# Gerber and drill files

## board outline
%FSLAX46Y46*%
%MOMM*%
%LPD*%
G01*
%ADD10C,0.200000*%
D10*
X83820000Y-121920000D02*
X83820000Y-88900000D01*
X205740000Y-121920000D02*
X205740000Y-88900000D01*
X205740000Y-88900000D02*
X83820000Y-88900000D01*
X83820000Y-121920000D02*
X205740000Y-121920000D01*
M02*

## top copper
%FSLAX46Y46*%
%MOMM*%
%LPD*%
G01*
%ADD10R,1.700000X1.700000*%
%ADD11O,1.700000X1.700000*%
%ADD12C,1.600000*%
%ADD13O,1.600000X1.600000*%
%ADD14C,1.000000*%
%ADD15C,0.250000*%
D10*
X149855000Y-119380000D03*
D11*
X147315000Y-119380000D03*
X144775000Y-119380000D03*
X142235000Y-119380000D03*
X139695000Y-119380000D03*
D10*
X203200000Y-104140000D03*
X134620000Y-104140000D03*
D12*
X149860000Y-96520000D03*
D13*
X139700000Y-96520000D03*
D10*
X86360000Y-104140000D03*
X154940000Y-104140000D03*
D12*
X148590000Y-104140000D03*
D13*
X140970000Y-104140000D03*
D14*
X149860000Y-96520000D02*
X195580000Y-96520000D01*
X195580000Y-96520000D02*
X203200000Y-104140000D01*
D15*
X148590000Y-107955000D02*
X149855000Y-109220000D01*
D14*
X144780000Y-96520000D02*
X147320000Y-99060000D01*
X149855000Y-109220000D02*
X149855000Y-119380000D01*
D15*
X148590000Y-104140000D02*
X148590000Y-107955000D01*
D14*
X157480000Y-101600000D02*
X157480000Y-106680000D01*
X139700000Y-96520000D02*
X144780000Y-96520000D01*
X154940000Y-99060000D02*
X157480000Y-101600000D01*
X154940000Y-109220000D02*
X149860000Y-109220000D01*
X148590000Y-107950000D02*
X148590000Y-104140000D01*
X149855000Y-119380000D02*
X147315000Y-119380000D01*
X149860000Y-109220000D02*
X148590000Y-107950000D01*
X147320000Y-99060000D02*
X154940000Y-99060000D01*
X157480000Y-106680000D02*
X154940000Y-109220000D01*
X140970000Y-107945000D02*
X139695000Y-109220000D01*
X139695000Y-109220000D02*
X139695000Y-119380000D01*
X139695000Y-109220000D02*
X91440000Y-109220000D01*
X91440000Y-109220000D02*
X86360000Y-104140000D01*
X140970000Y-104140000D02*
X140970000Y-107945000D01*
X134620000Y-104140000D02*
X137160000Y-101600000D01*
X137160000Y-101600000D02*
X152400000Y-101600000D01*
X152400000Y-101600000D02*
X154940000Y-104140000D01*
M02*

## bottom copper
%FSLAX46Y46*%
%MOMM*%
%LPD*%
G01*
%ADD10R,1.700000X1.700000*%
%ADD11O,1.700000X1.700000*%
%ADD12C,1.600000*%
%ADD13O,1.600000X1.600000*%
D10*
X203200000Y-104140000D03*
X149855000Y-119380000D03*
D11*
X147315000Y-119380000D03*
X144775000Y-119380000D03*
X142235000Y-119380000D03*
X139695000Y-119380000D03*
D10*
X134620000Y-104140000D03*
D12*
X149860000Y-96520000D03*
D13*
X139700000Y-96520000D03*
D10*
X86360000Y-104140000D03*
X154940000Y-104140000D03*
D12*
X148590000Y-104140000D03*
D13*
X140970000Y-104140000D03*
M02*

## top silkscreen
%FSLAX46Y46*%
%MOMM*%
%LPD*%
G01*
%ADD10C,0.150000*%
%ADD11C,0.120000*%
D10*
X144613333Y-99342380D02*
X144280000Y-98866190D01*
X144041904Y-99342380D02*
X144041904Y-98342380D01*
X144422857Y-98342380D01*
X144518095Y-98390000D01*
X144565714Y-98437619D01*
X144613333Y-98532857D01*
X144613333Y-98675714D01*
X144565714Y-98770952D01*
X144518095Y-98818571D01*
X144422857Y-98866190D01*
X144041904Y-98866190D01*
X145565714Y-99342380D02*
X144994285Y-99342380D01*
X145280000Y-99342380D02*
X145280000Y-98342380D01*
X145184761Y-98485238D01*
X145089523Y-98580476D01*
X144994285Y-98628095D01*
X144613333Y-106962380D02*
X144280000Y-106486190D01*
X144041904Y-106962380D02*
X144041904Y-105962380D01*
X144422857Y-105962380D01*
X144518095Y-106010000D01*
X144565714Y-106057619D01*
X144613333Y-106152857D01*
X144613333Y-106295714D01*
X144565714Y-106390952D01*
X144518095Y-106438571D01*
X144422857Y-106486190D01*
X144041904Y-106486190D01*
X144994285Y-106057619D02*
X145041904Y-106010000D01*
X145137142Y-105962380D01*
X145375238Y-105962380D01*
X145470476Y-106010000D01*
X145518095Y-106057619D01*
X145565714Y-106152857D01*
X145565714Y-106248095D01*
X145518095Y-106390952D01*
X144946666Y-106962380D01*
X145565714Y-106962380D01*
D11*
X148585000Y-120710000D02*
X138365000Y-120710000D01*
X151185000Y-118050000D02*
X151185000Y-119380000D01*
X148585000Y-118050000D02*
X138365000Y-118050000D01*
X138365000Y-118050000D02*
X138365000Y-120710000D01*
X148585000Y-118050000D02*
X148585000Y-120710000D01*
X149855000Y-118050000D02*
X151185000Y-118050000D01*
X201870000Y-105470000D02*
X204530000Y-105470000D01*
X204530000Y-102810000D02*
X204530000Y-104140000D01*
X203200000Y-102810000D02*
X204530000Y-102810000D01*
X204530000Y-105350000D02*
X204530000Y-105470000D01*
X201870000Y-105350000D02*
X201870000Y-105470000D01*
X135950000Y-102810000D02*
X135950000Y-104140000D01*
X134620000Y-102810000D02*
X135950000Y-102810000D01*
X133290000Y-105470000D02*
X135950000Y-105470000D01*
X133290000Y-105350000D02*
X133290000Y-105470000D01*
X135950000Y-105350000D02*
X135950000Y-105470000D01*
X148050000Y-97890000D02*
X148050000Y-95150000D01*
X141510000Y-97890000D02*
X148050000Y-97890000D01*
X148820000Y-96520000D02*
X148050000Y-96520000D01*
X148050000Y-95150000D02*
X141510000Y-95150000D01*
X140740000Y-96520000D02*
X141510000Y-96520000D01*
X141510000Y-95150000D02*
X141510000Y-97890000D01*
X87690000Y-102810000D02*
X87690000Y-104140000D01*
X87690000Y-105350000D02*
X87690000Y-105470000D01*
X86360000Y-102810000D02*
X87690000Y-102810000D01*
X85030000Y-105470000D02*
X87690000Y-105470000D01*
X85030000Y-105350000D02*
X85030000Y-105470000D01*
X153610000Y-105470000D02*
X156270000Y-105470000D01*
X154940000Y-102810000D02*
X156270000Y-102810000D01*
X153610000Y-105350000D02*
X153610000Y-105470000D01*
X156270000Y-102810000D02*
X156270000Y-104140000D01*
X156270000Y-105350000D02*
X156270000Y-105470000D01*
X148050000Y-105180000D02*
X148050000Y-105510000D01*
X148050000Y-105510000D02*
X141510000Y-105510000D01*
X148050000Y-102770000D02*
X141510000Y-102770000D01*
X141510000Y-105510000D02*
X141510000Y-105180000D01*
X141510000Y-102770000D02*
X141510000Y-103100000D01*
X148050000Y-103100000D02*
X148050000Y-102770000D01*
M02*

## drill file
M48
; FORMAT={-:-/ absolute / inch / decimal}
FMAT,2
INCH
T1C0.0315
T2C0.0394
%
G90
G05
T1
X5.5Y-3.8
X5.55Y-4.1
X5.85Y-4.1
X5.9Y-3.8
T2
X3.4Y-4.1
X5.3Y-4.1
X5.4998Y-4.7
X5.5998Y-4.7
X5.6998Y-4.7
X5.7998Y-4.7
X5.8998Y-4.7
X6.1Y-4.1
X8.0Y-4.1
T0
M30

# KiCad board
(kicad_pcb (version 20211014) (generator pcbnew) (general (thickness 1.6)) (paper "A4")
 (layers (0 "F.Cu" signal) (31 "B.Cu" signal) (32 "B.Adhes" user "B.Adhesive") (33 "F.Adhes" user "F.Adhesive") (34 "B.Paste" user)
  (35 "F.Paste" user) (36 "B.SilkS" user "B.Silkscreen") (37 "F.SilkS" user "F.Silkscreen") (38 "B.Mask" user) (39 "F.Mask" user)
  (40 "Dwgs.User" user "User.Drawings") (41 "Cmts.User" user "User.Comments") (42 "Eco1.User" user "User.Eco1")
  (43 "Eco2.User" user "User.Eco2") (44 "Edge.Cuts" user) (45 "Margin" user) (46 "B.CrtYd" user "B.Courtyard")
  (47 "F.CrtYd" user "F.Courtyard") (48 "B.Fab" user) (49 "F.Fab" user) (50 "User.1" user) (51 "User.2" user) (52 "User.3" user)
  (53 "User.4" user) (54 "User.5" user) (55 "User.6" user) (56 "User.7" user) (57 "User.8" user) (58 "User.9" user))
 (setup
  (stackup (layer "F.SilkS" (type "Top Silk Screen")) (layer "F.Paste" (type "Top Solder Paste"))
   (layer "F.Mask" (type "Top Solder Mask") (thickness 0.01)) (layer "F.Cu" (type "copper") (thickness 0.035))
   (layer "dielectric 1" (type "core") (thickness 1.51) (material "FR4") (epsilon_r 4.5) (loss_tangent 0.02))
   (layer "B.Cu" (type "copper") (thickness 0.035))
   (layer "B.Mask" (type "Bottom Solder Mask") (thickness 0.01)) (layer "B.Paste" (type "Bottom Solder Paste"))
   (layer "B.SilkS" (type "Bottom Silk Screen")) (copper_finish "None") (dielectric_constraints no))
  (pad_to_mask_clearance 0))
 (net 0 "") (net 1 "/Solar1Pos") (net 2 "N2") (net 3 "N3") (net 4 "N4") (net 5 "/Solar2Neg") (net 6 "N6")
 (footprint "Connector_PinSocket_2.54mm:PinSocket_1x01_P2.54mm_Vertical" (layer "F.Cu") (at 203.2 104.14)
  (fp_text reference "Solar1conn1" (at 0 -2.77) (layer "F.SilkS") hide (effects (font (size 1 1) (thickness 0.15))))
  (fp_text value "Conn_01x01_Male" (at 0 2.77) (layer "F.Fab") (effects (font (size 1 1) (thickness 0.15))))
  (fp_line (start -1.33 1.33) (end 1.33 1.33) (layer "F.SilkS") (width 0.12))
  (fp_line (start 1.33 -1.33) (end 1.33 0) (layer "F.SilkS") (width 0.12))
  (fp_line (start 0 -1.33) (end 1.33 -1.33) (layer "F.SilkS") (width 0.12))
  (fp_line (start 1.33 1.21) (end 1.33 1.33) (layer "F.SilkS") (width 0.12))
  (fp_line (start -1.33 1.21) (end -1.33 1.33) (layer "F.SilkS") (width 0.12))
  (pad "1" thru_hole rect (at 0 0) (size 1.7 1.7) (drill 1) (layers *.Cu *.Mask) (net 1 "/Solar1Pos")))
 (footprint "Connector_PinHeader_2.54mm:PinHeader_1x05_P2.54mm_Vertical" (layer "F.Cu") (at 149.855 119.38 -90)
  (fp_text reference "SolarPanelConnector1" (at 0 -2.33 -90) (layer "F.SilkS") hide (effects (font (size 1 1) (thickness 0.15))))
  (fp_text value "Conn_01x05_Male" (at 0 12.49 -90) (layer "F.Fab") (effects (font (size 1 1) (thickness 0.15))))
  (fp_line (start -1.33 0) (end -1.33 -1.33) (layer "F.SilkS") (width 0.12))
  (fp_line (start 1.33 1.27) (end 1.33 11.49) (layer "F.SilkS") (width 0.12))
  (fp_line (start -1.33 11.49) (end 1.33 11.49) (layer "F.SilkS") (width 0.12))
  (fp_line (start -1.33 1.27) (end -1.33 11.49) (layer "F.SilkS") (width 0.12))
  (fp_line (start -1.33 1.27) (end 1.33 1.27) (layer "F.SilkS") (width 0.12))
  (fp_line (start -1.33 -1.33) (end 0 -1.33) (layer "F.SilkS") (width 0.12))
  (pad "1" thru_hole rect (at 0 0 270) (size 1.7 1.7) (drill 1) (layers *.Cu *.Mask) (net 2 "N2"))
  (pad "2" thru_hole oval (at 0 2.54 270) (size 1.7 1.7) (drill 1) (layers *.Cu *.Mask) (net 2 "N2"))
  (pad "3" thru_hole oval (at 0 5.08 270) (size 1.7 1.7) (drill 1) (layers *.Cu *.Mask) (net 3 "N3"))
  (pad "4" thru_hole oval (at 0 7.62 270) (size 1.7 1.7) (drill 1) (layers *.Cu *.Mask) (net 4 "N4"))
  (pad "5" thru_hole oval (at 0 10.16 270) (size 1.7 1.7) (drill 1) (layers *.Cu *.Mask) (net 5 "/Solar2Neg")))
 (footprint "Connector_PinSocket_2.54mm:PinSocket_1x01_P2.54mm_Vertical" (layer "F.Cu") (at 134.62 104.14)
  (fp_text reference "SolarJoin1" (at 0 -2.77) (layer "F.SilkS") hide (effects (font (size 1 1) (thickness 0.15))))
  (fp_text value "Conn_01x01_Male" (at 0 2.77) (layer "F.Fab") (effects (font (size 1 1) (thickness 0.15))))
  (fp_line (start 1.33 -1.33) (end 1.33 0) (layer "F.SilkS") (width 0.12))
  (fp_line (start 0 -1.33) (end 1.33 -1.33) (layer "F.SilkS") (width 0.12))
  (fp_line (start -1.33 1.33) (end 1.33 1.33) (layer "F.SilkS") (width 0.12))
  (fp_line (start -1.33 1.21) (end -1.33 1.33) (layer "F.SilkS") (width 0.12))
  (fp_line (start 1.33 1.21) (end 1.33 1.33) (layer "F.SilkS") (width 0.12))
  (pad "1" thru_hole rect (at 0 0) (size 1.7 1.7) (drill 1) (layers *.Cu *.Mask) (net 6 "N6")))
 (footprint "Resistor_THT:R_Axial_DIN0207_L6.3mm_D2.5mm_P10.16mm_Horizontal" (layer "F.Cu") (at 149.86 96.52 180)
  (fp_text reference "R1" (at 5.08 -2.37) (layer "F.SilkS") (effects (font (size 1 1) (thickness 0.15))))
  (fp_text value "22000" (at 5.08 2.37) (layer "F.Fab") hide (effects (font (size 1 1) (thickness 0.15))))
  (fp_line (start 1.81 -1.37) (end 1.81 1.37) (layer "F.SilkS") (width 0.12))
  (fp_line (start 8.35 -1.37) (end 1.81 -1.37) (layer "F.SilkS") (width 0.12))
  (fp_line (start 1.04 0) (end 1.81 0) (layer "F.SilkS") (width 0.12))
  (fp_line (start 1.81 1.37) (end 8.35 1.37) (layer "F.SilkS") (width 0.12))
  (fp_line (start 9.12 0) (end 8.35 0) (layer "F.SilkS") (width 0.12))
  (fp_line (start 8.35 1.37) (end 8.35 -1.37) (layer "F.SilkS") (width 0.12))
  (pad "1" thru_hole circle (at 0 0 180) (size 1.6 1.6) (drill 0.8) (layers *.Cu *.Mask) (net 1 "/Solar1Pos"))
  (pad "2" thru_hole oval (at 10.16 0 180) (size 1.6 1.6) (drill 0.8) (layers *.Cu *.Mask) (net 2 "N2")))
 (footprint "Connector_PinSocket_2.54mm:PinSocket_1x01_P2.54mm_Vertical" (layer "F.Cu") (at 86.36 104.14)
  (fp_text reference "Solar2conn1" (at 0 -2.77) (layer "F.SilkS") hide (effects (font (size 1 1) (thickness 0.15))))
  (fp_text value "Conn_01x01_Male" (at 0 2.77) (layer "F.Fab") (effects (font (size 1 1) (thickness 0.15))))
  (fp_line (start 1.33 -1.33) (end 1.33 0) (layer "F.SilkS") (width 0.12))
  (fp_line (start 1.33 1.21) (end 1.33 1.33) (layer "F.SilkS") (width 0.12))
  (fp_line (start 0 -1.33) (end 1.33 -1.33) (layer "F.SilkS") (width 0.12))
  (fp_line (start -1.33 1.33) (end 1.33 1.33) (layer "F.SilkS") (width 0.12))
  (fp_line (start -1.33 1.21) (end -1.33 1.33) (layer "F.SilkS") (width 0.12))
  (pad "1" thru_hole rect (at 0 0) (size 1.7 1.7) (drill 1) (layers *.Cu *.Mask) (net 5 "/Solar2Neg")))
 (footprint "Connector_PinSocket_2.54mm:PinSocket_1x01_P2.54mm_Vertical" (layer "F.Cu") (at 154.94 104.14)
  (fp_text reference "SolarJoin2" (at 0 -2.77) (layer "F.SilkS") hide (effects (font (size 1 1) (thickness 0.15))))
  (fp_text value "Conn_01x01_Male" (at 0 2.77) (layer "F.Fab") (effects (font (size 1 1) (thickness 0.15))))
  (fp_line (start -1.33 1.33) (end 1.33 1.33) (layer "F.SilkS") (width 0.12))
  (fp_line (start 0 -1.33) (end 1.33 -1.33) (layer "F.SilkS") (width 0.12))
  (fp_line (start -1.33 1.21) (end -1.33 1.33) (layer "F.SilkS") (width 0.12))
  (fp_line (start 1.33 -1.33) (end 1.33 0) (layer "F.SilkS") (width 0.12))
  (fp_line (start 1.33 1.21) (end 1.33 1.33) (layer "F.SilkS") (width 0.12))
  (pad "1" thru_hole rect (at 0 0) (size 1.7 1.7) (drill 1) (layers *.Cu *.Mask) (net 6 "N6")))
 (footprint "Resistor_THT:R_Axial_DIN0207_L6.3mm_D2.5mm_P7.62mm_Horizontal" (layer "F.Cu") (at 148.59 104.14 180)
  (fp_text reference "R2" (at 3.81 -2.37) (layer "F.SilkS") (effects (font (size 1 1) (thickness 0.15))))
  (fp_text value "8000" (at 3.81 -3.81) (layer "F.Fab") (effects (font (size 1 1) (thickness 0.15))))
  (fp_line (start 0.54 -1.04) (end 0.54 -1.37) (layer "F.SilkS") (width 0.12))
  (fp_line (start 0.54 -1.37) (end 7.08 -1.37) (layer "F.SilkS") (width 0.12))
  (fp_line (start 0.54 1.37) (end 7.08 1.37) (layer "F.SilkS") (width 0.12))
  (fp_line (start 7.08 -1.37) (end 7.08 -1.04) (layer "F.SilkS") (width 0.12))
  (fp_line (start 7.08 1.37) (end 7.08 1.04) (layer "F.SilkS") (width 0.12))
  (fp_line (start 0.54 1.04) (end 0.54 1.37) (layer "F.SilkS") (width 0.12))
  (pad "1" thru_hole circle (at 0 0 180) (size 1.6 1.6) (drill 0.8) (layers *.Cu *.Mask) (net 2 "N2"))
  (pad "2" thru_hole oval (at 7.62 0 180) (size 1.6 1.6) (drill 0.8) (layers *.Cu *.Mask) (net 5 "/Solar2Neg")))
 (gr_line (start 83.82 121.92) (end 83.82 88.9) (layer "Edge.Cuts") (width 0.2))
 (gr_line (start 205.74 121.92) (end 205.74 88.9) (layer "Edge.Cuts") (width 0.2))
 (gr_line (start 205.74 88.9) (end 83.82 88.9) (layer "Edge.Cuts") (width 0.2))
 (gr_line (start 83.82 121.92) (end 205.74 121.92) (layer "Edge.Cuts") (width 0.2))
 (segment (start 149.86 96.52) (end 195.58 96.52) (width 1) (layer "F.Cu") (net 1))
 (segment (start 195.58 96.52) (end 203.2 104.14) (width 1) (layer "F.Cu") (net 1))
 (segment (start 148.59 107.955) (end 149.855 109.22) (width 0.25) (layer "F.Cu") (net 2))
 (segment (start 144.78 96.52) (end 147.32 99.06) (width 1) (layer "F.Cu") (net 2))
 (segment (start 149.855 109.22) (end 149.855 119.38) (width 1) (layer "F.Cu") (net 2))
 (segment (start 148.59 104.14) (end 148.59 107.955) (width 0.25) (layer "F.Cu") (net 2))
 (segment (start 157.48 101.6) (end 157.48 106.68) (width 1) (layer "F.Cu") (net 2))
 (segment (start 139.7 96.52) (end 144.78 96.52) (width 1) (layer "F.Cu") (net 2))
 (segment (start 154.94 99.06) (end 157.48 101.6) (width 1) (layer "F.Cu") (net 2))
 (segment (start 154.94 109.22) (end 149.86 109.22) (width 1) (layer "F.Cu") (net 2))
 (segment (start 148.59 107.95) (end 148.59 104.14) (width 1) (layer "F.Cu") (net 2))
 (segment (start 149.855 119.38) (end 147.315 119.38) (width 1) (layer "F.Cu") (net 2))
 (segment (start 149.86 109.22) (end 148.59 107.95) (width 1) (layer "F.Cu") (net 2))
 (segment (start 147.32 99.06) (end 154.94 99.06) (width 1) (layer "F.Cu") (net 2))
 (segment (start 157.48 106.68) (end 154.94 109.22) (width 1) (layer "F.Cu") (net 2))
 (segment (start 140.97 107.945) (end 139.695 109.22) (width 1) (layer "F.Cu") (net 5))
 (segment (start 139.695 109.22) (end 139.695 119.38) (width 1) (layer "F.Cu") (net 5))
 (segment (start 139.695 109.22) (end 91.44 109.22) (width 1) (layer "F.Cu") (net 5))
 (segment (start 91.44 109.22) (end 86.36 104.14) (width 1) (layer "F.Cu") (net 5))
 (segment (start 140.97 104.14) (end 140.97 107.945) (width 1) (layer "F.Cu") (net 5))
 (segment (start 134.62 104.14) (end 137.16 101.6) (width 1) (layer "F.Cu") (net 6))
 (segment (start 137.16 101.6) (end 152.4 101.6) (width 1) (layer "F.Cu") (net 6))
 (segment (start 152.4 101.6) (end 154.94 104.14) (width 1) (layer "F.Cu") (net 6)))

